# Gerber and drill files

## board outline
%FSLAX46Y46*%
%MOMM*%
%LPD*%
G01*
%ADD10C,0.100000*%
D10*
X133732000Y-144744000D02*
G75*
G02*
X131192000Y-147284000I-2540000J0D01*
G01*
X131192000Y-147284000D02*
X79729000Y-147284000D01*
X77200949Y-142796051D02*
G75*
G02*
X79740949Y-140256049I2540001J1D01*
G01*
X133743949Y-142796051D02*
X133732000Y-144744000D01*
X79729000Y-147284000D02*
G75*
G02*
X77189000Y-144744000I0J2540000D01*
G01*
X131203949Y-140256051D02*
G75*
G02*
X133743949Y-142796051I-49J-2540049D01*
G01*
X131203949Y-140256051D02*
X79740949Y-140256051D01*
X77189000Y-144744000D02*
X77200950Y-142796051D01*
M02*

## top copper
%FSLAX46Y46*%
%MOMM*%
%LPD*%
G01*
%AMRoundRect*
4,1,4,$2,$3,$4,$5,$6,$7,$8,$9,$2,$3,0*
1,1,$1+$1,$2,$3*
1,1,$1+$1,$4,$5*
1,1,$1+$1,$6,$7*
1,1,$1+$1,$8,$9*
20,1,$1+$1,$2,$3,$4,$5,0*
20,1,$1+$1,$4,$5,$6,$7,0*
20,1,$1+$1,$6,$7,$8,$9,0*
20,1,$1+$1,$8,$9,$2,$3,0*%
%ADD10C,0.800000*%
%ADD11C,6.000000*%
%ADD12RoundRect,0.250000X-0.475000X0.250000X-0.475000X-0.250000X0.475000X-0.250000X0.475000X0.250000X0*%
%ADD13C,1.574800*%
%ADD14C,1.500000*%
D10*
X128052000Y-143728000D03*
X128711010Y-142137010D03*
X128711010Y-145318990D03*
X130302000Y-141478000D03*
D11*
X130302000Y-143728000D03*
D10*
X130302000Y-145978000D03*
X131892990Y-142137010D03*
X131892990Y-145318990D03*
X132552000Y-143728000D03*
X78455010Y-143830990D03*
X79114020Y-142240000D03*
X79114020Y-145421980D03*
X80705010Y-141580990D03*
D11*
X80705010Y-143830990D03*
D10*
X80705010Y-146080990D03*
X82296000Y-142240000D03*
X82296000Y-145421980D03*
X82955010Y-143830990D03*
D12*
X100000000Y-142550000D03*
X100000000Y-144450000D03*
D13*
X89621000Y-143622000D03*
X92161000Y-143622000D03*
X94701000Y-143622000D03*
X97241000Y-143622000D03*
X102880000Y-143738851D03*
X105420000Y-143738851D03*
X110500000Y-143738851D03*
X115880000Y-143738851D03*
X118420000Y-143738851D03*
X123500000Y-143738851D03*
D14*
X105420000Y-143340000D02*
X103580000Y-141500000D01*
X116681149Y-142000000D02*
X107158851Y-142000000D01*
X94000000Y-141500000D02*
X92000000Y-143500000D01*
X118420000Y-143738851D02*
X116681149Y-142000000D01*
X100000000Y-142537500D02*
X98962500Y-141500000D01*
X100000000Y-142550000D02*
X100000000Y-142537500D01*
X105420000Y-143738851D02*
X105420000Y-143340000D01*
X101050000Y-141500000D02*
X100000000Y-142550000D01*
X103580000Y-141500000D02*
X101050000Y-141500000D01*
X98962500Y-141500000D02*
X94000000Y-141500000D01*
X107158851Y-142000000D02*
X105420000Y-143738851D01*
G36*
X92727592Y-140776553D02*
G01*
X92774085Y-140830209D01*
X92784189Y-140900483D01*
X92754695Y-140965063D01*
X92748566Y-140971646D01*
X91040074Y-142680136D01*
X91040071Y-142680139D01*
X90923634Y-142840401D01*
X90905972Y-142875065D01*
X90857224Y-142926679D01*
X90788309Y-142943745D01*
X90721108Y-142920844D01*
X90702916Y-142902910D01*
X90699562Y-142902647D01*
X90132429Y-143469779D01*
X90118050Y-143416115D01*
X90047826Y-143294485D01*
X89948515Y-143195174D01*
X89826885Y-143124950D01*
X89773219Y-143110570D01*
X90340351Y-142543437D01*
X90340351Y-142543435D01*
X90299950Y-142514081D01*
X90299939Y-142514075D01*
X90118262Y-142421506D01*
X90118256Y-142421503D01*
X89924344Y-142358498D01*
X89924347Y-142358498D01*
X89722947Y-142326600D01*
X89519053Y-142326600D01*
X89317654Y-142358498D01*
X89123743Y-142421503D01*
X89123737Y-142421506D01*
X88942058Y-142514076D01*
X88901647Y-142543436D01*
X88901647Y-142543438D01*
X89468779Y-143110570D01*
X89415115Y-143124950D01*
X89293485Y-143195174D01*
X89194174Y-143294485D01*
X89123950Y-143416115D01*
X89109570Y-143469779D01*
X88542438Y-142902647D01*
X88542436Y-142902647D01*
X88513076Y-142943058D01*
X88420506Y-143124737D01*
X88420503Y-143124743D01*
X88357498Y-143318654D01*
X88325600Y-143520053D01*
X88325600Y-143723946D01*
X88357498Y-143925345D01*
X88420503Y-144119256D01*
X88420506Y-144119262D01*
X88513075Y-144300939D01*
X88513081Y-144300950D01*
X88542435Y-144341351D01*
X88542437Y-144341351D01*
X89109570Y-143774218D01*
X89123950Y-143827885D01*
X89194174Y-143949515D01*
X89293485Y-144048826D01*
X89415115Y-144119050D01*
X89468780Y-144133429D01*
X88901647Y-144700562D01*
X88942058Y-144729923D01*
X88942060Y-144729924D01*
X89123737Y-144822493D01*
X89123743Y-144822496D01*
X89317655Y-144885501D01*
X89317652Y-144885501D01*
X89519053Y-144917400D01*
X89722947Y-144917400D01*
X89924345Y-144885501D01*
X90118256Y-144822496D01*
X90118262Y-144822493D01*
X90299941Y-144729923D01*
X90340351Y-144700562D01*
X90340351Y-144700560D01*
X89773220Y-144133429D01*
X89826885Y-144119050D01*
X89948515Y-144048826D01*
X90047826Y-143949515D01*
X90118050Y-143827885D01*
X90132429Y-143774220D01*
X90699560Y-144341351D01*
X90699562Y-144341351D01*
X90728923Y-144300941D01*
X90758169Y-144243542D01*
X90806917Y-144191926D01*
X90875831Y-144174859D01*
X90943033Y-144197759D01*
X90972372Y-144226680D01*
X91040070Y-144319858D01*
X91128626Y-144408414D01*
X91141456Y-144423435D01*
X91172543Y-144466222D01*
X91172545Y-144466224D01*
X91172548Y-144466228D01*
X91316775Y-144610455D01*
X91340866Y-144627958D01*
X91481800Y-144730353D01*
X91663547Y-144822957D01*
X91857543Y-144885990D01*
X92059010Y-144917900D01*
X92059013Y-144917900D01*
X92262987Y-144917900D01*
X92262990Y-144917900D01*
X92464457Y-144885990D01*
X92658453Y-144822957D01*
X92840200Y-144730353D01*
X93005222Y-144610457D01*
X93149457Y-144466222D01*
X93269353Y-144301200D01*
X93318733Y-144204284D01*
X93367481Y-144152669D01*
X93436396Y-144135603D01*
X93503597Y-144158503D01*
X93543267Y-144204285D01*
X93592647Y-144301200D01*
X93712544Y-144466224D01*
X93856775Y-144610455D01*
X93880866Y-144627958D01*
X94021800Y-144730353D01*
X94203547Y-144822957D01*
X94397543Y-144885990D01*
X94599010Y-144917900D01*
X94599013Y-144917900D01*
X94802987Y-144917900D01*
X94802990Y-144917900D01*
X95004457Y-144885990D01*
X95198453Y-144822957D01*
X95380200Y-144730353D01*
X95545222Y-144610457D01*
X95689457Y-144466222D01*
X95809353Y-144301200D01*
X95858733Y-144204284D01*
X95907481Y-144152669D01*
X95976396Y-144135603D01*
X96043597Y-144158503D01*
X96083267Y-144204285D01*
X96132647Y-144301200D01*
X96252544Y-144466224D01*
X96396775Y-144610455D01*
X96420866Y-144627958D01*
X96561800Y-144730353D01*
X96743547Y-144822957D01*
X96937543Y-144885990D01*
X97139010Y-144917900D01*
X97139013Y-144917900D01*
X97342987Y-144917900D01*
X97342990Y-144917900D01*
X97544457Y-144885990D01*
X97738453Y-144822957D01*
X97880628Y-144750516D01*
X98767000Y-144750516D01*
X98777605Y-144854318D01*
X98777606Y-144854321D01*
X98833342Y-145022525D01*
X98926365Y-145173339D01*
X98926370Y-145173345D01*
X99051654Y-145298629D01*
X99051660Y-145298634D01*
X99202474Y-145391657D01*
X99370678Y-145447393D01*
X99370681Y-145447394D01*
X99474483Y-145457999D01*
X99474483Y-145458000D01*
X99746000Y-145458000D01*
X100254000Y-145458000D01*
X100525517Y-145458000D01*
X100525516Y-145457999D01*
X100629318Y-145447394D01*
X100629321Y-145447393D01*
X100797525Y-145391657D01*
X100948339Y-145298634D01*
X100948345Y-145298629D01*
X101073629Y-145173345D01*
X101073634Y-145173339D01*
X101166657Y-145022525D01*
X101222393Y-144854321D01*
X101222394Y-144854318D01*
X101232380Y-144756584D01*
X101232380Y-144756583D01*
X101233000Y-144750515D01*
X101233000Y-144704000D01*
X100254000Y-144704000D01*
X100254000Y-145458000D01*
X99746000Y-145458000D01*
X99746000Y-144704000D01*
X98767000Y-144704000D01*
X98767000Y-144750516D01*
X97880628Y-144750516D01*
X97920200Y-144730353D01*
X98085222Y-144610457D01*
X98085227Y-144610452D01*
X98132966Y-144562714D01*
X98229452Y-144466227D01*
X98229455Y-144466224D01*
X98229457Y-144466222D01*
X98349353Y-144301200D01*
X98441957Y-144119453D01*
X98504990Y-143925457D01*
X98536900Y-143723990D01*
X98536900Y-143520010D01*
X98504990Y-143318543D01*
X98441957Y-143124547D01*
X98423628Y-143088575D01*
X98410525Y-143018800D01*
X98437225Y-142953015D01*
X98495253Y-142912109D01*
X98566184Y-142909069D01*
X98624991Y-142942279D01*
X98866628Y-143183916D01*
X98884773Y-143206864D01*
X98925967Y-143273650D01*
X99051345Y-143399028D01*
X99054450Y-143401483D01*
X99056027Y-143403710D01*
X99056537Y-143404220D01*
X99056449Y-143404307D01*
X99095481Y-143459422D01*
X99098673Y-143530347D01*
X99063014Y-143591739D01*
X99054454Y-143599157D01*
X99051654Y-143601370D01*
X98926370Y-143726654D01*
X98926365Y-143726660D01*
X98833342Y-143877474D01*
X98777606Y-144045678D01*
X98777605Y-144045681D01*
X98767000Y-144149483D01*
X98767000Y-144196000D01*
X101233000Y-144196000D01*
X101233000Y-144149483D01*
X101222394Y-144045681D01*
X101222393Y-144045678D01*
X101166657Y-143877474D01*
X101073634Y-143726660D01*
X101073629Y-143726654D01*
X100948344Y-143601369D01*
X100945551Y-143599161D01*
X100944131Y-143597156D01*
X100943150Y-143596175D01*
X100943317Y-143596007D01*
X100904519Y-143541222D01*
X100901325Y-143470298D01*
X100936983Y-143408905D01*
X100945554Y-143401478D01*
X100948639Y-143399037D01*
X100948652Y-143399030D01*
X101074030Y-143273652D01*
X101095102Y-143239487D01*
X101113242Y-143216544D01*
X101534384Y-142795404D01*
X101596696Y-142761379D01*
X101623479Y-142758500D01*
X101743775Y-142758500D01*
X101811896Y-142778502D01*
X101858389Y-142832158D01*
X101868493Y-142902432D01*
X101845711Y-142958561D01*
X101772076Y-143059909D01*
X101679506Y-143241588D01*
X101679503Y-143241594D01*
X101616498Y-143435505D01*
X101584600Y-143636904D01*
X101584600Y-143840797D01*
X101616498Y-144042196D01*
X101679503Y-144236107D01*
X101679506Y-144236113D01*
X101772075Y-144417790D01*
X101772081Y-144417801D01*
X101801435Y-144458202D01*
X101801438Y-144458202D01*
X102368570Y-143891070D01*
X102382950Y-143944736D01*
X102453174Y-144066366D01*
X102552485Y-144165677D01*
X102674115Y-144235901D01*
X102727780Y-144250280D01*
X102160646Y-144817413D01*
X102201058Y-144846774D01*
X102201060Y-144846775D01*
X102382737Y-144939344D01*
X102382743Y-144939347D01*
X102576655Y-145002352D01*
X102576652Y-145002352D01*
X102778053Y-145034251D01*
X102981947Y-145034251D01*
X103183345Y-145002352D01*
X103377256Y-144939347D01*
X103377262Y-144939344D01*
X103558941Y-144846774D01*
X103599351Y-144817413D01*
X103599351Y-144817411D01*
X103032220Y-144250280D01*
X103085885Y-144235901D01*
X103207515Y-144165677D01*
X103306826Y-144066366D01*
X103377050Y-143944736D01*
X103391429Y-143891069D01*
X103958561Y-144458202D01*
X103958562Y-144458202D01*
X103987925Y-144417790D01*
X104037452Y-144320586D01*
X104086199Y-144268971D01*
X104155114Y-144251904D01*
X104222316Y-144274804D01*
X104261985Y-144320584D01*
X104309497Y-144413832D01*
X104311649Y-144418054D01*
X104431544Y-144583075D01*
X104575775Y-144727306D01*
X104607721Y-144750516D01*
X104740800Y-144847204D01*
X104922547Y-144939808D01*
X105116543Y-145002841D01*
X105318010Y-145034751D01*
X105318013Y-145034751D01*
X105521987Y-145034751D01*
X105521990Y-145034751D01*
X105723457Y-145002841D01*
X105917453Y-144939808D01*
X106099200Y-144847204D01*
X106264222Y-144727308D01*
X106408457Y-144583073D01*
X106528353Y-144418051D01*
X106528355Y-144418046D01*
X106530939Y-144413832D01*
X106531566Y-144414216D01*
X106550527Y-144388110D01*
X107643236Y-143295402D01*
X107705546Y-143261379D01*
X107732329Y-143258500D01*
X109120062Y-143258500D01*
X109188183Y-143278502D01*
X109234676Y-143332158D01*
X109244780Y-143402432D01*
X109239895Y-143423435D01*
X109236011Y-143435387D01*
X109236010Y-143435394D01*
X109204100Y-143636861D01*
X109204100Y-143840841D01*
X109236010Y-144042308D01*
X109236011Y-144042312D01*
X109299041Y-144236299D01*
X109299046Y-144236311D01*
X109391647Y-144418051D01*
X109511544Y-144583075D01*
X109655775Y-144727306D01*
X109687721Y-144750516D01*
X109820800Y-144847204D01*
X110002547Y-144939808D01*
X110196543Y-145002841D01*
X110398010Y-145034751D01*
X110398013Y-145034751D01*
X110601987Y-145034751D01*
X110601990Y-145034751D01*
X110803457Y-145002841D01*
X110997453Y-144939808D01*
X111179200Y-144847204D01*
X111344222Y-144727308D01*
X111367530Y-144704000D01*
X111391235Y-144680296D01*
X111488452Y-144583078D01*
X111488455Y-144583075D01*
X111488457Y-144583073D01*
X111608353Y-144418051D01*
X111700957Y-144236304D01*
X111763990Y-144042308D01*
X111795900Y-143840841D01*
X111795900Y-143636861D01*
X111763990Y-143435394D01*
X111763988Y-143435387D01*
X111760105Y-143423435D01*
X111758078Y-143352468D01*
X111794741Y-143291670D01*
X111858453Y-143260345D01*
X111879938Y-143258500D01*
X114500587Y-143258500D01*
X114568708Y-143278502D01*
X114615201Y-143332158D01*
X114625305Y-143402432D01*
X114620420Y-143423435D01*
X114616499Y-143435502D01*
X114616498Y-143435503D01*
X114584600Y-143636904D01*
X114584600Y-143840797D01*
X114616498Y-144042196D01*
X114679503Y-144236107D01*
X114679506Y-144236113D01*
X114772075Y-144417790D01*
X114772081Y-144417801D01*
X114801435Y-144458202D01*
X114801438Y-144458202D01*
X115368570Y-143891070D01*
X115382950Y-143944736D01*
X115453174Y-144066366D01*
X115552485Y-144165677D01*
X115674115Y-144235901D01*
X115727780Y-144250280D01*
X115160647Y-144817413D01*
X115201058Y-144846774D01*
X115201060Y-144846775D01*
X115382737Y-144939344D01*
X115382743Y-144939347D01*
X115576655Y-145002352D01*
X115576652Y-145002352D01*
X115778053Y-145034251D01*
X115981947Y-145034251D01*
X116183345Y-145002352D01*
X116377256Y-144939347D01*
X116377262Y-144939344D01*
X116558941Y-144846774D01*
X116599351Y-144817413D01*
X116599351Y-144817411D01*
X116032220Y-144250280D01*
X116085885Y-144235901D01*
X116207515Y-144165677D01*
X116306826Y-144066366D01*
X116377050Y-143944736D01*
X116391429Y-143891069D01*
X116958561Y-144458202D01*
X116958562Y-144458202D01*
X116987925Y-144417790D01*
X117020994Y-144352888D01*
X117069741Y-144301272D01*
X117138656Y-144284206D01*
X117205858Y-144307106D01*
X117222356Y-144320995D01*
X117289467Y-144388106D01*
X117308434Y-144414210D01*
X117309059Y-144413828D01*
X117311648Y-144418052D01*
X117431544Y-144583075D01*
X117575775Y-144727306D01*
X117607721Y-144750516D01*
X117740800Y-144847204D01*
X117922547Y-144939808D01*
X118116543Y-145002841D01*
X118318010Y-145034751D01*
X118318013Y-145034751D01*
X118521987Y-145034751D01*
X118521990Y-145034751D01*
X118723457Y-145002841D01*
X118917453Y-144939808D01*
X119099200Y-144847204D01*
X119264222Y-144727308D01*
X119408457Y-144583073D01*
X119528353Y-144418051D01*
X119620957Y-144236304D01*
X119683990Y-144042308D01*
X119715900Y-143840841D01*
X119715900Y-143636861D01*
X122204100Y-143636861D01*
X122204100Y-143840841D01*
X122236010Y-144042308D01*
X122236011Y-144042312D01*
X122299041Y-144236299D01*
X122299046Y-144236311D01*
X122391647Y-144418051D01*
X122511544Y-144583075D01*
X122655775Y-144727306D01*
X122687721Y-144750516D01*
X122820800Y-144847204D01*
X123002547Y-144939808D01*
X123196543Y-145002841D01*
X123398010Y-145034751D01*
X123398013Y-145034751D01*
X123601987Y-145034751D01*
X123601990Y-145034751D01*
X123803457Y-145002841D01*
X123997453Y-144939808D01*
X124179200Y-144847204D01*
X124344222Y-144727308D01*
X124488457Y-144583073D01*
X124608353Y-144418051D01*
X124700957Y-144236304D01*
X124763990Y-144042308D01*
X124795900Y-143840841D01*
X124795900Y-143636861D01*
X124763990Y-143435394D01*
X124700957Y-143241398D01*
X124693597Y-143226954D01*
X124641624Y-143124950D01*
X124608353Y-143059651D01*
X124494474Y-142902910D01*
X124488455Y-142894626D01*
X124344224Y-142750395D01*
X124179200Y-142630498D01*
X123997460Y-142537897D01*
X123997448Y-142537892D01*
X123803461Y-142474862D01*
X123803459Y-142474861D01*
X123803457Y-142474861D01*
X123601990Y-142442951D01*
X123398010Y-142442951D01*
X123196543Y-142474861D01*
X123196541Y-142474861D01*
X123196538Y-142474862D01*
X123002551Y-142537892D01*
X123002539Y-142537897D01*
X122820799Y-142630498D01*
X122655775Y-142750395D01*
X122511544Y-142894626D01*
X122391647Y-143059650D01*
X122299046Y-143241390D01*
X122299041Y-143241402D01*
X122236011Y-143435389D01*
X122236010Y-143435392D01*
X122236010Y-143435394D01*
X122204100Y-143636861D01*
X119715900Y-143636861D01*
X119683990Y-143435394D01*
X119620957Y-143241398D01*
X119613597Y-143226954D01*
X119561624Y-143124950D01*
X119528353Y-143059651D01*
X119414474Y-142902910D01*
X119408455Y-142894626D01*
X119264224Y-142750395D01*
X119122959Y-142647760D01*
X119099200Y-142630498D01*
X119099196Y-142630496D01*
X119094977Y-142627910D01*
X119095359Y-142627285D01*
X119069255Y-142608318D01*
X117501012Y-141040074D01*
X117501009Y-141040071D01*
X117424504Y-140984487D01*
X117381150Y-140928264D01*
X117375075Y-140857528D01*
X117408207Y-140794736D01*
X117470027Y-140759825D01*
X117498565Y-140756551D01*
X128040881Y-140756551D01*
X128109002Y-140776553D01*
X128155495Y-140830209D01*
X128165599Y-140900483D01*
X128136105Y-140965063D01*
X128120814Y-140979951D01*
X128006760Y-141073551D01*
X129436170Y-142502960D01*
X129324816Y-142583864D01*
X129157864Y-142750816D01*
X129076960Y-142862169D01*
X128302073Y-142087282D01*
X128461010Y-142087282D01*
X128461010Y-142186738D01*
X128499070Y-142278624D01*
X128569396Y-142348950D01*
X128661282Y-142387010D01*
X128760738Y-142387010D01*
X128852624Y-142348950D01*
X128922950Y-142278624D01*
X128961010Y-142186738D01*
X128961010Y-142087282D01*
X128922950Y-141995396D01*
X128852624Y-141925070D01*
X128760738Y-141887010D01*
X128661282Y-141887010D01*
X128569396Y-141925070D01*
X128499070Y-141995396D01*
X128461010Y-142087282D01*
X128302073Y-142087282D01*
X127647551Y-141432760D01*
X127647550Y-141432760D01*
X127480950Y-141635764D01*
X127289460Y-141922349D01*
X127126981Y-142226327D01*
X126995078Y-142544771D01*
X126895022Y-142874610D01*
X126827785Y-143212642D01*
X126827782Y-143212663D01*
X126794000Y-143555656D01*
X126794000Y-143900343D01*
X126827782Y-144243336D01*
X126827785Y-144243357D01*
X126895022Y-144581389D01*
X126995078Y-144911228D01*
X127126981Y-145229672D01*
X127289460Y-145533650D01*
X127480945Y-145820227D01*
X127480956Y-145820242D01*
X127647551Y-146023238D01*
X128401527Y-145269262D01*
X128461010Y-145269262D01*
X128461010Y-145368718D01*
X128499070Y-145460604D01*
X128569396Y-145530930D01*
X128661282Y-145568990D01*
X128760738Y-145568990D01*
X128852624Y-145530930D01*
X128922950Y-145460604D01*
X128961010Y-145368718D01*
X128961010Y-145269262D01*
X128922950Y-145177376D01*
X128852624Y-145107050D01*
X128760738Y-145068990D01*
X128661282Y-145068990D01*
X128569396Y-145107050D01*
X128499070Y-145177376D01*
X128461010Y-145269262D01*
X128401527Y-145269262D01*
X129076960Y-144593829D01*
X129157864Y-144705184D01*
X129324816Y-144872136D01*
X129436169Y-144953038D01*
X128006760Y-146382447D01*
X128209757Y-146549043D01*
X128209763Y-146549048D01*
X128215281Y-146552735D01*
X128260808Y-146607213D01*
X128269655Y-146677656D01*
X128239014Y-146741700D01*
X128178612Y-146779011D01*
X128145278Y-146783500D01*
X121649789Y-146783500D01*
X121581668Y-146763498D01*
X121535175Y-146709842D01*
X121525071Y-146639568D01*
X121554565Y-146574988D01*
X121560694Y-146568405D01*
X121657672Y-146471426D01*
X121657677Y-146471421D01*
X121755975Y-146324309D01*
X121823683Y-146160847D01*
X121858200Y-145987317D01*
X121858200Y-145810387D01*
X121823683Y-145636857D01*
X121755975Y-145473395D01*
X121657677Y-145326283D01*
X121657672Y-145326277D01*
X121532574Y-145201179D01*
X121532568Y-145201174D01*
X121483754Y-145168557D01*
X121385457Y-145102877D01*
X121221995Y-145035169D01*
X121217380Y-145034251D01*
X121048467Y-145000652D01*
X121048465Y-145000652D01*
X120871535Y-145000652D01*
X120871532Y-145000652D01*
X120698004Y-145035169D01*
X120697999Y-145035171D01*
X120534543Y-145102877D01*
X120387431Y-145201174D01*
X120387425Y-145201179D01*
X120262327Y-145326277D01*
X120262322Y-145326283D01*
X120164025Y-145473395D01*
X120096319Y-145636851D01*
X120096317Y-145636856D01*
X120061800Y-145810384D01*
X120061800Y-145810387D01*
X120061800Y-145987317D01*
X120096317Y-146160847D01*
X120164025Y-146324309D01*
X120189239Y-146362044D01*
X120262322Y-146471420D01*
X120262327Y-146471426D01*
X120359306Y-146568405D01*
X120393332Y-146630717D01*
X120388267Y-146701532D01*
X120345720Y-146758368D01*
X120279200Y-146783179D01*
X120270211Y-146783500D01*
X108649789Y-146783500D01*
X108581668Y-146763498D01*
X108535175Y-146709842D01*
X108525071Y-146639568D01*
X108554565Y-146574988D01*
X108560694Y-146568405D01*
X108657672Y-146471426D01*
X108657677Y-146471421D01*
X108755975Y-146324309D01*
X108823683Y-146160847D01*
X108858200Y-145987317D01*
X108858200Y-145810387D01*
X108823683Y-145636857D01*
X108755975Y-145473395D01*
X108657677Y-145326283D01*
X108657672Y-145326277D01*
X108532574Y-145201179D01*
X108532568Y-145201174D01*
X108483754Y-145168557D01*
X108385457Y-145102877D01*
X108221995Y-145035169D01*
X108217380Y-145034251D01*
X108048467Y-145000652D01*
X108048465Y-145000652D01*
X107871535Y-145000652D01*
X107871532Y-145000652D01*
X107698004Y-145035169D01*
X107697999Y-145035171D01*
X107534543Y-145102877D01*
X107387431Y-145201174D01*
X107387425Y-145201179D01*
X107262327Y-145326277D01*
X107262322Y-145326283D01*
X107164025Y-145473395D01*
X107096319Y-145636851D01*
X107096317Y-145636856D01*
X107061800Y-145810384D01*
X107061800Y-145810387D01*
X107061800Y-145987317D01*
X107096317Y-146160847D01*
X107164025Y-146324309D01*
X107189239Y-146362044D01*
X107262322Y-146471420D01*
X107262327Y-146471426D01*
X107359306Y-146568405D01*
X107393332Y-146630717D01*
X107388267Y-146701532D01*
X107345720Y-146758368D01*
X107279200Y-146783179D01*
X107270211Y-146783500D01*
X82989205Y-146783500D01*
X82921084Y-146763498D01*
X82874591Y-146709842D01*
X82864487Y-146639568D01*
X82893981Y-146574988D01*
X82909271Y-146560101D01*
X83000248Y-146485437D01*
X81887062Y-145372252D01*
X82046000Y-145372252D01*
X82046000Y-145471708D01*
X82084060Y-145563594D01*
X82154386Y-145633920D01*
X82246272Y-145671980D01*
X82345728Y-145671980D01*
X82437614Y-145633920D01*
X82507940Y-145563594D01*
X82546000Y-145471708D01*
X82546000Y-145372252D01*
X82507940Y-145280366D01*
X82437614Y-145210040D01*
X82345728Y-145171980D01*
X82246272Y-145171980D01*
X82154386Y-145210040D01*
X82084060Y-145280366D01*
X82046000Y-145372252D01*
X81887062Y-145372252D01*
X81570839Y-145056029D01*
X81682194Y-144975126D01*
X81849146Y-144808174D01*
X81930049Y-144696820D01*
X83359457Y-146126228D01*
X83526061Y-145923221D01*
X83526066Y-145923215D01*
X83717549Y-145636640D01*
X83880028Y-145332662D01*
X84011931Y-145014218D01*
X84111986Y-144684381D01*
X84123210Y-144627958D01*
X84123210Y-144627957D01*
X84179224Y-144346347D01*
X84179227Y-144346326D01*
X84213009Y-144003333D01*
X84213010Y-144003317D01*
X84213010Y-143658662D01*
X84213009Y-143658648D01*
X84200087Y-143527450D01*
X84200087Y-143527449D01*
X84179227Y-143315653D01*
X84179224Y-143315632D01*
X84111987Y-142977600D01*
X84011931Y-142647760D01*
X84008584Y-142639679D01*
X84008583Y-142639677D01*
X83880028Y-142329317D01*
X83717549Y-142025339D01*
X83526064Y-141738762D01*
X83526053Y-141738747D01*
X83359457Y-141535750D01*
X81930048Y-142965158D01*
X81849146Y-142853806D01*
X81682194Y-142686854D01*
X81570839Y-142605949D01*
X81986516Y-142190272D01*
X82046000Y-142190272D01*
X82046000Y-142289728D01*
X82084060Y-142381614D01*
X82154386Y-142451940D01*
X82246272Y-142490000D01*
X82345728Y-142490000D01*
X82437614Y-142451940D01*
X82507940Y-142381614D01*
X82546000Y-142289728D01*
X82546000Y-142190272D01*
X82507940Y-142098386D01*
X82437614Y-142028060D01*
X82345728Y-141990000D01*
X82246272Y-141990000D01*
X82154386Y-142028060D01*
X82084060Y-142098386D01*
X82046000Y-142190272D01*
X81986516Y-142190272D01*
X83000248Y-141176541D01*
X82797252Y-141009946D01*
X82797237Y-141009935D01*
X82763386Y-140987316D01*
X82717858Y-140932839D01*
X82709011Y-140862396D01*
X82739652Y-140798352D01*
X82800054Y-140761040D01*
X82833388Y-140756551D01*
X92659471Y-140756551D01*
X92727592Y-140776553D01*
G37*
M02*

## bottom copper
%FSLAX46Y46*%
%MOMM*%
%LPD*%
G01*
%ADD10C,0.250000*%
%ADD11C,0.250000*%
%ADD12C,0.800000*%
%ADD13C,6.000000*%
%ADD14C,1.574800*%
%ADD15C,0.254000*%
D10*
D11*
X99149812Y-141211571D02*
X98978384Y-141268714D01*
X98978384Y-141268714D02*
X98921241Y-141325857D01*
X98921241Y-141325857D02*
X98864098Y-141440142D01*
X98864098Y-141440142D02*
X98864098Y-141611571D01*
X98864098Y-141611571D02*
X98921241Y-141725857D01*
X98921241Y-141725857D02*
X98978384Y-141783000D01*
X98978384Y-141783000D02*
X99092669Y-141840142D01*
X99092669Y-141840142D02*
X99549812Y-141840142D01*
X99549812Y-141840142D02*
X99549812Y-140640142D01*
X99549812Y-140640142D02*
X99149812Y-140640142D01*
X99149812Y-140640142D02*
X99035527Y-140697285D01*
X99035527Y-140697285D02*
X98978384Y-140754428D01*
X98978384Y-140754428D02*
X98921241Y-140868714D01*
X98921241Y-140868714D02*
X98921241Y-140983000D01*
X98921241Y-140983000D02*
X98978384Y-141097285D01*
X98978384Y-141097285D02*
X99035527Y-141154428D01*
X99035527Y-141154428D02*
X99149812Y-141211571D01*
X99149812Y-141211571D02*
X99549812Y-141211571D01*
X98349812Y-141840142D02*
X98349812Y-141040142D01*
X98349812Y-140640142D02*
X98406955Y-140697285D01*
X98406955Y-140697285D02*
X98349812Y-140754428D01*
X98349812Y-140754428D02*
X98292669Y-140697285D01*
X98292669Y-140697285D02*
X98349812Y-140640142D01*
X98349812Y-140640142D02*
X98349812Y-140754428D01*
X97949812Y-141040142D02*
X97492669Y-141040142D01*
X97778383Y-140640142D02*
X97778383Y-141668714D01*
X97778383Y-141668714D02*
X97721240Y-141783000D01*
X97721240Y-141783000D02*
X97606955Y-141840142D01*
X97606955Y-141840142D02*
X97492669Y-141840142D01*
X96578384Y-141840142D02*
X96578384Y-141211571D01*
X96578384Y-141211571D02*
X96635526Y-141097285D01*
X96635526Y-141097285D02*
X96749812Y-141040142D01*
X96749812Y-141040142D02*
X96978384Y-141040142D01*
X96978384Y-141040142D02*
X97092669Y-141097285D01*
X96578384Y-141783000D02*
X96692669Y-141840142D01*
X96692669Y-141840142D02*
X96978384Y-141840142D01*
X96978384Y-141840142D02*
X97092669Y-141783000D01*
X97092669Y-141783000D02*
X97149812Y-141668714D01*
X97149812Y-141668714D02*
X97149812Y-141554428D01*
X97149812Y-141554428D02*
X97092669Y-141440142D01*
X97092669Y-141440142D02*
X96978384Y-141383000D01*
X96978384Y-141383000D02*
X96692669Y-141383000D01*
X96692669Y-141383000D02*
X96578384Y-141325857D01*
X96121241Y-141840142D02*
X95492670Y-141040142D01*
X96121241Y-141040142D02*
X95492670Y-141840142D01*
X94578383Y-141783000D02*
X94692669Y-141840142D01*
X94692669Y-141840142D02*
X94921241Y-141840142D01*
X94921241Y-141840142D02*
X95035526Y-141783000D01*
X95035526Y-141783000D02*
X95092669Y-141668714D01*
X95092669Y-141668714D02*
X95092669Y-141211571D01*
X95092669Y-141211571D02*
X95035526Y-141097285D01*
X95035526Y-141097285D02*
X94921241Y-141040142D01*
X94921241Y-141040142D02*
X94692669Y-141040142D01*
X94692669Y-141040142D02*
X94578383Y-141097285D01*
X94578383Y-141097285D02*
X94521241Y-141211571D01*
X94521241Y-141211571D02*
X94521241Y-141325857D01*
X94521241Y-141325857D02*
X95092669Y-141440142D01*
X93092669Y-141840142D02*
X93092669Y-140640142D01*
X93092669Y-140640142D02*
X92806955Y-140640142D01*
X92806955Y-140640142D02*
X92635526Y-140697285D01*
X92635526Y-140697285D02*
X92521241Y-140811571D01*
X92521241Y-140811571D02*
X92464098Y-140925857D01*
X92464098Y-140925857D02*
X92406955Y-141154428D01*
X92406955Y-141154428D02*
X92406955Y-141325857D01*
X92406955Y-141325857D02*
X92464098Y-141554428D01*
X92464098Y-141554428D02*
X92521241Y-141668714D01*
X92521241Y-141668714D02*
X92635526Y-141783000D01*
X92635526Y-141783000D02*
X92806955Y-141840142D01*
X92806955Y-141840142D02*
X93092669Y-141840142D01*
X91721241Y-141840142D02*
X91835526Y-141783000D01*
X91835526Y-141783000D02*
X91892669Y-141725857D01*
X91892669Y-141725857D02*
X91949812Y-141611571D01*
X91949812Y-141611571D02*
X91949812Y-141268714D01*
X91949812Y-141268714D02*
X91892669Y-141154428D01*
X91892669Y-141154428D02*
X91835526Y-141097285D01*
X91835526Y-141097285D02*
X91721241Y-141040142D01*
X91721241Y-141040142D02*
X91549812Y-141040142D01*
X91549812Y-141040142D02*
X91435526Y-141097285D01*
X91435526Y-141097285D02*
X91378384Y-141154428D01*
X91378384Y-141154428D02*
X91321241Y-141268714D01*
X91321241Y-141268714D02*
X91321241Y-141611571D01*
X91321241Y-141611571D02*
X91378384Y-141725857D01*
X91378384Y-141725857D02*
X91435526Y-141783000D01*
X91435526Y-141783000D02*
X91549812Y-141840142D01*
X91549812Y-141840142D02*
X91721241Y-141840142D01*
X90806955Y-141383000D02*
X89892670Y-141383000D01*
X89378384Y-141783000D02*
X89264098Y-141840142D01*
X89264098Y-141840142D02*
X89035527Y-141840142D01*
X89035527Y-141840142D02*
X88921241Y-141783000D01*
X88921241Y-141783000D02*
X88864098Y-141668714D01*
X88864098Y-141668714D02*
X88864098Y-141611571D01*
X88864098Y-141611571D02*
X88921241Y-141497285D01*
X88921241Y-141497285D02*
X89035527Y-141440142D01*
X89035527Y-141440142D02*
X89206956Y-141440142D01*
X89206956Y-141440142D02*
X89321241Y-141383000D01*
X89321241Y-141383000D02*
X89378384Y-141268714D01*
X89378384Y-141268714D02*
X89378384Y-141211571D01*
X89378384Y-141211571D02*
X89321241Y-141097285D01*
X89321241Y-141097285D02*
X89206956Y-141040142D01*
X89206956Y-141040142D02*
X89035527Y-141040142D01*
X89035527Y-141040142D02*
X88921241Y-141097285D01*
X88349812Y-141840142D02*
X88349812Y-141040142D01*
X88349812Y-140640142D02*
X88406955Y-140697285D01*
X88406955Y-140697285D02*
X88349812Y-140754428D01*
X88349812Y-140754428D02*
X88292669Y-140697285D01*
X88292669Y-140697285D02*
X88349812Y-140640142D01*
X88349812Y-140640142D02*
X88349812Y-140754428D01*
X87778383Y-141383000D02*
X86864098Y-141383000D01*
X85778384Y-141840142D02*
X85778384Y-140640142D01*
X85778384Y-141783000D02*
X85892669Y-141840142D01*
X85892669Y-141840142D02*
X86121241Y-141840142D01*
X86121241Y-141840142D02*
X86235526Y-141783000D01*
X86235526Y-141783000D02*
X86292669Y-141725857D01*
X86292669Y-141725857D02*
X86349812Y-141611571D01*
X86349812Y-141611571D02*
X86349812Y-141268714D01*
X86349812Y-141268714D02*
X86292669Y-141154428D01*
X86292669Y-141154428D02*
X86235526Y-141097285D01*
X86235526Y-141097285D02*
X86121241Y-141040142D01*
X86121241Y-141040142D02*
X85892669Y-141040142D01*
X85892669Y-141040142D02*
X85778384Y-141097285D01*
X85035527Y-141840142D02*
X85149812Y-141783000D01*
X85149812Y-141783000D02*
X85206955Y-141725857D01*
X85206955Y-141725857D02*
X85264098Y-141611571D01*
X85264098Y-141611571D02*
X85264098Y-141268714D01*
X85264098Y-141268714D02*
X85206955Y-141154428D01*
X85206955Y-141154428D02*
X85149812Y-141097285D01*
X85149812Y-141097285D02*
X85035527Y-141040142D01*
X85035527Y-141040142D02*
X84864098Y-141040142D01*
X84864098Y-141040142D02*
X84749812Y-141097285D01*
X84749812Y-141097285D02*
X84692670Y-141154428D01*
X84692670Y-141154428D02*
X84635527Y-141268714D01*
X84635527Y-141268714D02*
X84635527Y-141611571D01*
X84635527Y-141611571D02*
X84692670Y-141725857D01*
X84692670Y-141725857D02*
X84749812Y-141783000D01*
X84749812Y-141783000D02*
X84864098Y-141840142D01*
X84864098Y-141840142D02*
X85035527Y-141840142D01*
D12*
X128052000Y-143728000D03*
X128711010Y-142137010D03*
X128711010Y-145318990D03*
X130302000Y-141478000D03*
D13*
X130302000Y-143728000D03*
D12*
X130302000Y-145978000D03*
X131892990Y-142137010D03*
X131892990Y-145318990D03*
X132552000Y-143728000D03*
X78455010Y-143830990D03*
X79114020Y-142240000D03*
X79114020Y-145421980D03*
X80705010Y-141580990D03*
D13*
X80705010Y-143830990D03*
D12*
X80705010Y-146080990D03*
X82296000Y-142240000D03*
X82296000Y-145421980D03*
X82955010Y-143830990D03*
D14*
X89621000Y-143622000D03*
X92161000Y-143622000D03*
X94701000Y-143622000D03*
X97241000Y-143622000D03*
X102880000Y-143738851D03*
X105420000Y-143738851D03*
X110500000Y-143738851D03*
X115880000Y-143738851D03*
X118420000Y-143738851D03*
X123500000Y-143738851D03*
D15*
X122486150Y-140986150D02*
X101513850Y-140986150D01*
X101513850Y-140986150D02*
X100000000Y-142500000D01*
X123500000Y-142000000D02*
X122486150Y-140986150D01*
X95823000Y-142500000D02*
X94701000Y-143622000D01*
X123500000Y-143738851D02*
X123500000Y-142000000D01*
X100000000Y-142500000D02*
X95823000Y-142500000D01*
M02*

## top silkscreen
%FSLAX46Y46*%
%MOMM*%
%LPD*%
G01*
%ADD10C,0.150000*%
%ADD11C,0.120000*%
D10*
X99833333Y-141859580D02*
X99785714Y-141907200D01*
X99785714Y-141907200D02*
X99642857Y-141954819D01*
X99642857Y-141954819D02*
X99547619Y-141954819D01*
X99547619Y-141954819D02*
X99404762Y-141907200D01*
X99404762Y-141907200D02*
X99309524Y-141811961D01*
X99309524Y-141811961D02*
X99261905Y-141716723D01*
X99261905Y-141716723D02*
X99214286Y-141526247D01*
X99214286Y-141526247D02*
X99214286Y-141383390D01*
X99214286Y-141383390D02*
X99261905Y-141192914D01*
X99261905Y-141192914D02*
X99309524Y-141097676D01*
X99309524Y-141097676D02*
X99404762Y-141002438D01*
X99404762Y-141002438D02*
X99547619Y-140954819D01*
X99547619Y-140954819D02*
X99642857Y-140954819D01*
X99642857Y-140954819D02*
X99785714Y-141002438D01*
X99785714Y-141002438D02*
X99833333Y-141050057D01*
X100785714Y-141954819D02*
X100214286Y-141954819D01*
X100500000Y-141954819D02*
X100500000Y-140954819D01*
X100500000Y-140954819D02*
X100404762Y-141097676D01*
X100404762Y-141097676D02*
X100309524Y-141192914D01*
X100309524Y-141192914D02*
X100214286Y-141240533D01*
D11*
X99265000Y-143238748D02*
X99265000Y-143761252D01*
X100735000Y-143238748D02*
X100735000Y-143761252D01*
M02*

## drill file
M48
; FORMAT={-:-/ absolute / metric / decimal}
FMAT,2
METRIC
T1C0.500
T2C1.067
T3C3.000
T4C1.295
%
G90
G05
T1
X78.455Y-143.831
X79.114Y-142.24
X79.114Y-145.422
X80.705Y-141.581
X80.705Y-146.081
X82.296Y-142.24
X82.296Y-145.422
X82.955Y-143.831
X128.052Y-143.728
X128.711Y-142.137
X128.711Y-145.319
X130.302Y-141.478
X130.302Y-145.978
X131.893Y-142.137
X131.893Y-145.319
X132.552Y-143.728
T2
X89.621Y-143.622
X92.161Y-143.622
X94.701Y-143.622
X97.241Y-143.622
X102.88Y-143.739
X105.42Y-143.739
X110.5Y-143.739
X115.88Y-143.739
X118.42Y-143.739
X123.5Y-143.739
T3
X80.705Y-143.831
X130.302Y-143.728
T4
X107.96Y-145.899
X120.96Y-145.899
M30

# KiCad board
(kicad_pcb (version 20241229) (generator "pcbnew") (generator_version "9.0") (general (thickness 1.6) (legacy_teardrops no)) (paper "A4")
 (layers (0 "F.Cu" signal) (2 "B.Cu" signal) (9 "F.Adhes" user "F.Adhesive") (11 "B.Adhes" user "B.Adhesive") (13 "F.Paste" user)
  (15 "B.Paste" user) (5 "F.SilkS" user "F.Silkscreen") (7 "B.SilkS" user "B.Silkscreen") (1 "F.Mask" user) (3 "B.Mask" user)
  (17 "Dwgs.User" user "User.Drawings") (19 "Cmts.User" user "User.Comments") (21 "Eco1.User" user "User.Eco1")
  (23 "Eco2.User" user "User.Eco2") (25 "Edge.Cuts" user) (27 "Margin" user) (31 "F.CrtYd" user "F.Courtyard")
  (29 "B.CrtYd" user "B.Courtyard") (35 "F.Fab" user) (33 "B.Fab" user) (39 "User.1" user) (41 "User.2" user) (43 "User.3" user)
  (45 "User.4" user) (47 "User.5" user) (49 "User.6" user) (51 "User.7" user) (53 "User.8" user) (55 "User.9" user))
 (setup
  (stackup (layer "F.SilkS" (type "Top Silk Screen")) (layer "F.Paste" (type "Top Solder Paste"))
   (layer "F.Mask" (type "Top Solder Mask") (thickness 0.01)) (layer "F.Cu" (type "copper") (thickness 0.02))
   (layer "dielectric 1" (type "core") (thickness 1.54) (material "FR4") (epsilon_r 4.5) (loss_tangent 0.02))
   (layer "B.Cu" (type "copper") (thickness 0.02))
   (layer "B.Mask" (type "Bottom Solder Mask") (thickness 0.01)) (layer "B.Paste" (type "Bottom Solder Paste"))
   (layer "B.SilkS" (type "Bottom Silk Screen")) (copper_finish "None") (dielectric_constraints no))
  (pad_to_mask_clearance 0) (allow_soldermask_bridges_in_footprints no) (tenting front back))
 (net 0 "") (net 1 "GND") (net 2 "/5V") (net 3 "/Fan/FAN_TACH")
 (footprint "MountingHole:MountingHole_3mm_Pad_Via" (layer "F.Cu") (at 130.302 143.728)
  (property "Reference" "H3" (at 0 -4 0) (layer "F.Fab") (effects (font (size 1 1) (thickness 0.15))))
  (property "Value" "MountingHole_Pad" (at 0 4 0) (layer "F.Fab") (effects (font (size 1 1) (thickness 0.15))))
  (pad "1" thru_hole circle (at -2.25 0) (size 0.8 0.8) (drill 0.5) (layers "*.Cu" "*.Mask") (remove_unused_layers no) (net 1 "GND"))
  (pad "1" thru_hole circle (at -1.59099 -1.59099) (size 0.8 0.8) (drill 0.5) (layers "*.Cu" "*.Mask") (remove_unused_layers no)
   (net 1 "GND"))
  (pad "1" thru_hole circle (at -1.59099 1.59099) (size 0.8 0.8) (drill 0.5) (layers "*.Cu" "*.Mask") (remove_unused_layers no)
   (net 1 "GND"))
  (pad "1" thru_hole circle (at 0 -2.25) (size 0.8 0.8) (drill 0.5) (layers "*.Cu" "*.Mask") (remove_unused_layers no) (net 1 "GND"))
  (pad "1" thru_hole circle (at 0 0) (size 6 6) (drill 3) (layers "*.Cu" "*.Mask") (remove_unused_layers no) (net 1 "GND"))
  (pad "1" thru_hole circle (at 0 2.25) (size 0.8 0.8) (drill 0.5) (layers "*.Cu" "*.Mask") (remove_unused_layers no) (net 1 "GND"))
  (pad "1" thru_hole circle (at 1.59099 -1.59099) (size 0.8 0.8) (drill 0.5) (layers "*.Cu" "*.Mask") (remove_unused_layers no)
   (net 1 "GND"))
  (pad "1" thru_hole circle (at 1.59099 1.59099) (size 0.8 0.8) (drill 0.5) (layers "*.Cu" "*.Mask") (remove_unused_layers no) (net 1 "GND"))
  (pad "1" thru_hole circle (at 2.25 0) (size 0.8 0.8) (drill 0.5) (layers "*.Cu" "*.Mask") (remove_unused_layers no) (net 1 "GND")))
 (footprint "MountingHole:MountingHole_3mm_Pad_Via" (layer "F.Cu") (at 80.70501 143.83099)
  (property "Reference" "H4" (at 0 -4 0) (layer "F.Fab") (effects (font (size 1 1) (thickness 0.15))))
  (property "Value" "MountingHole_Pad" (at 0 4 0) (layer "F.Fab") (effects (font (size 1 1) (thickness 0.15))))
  (pad "1" thru_hole circle (at -2.25 0) (size 0.8 0.8) (drill 0.5) (layers "*.Cu" "*.Mask") (remove_unused_layers no) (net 1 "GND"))
  (pad "1" thru_hole circle (at -1.59099 -1.59099) (size 0.8 0.8) (drill 0.5) (layers "*.Cu" "*.Mask") (remove_unused_layers no)
   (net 1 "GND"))
  (pad "1" thru_hole circle (at -1.59099 1.59099) (size 0.8 0.8) (drill 0.5) (layers "*.Cu" "*.Mask") (remove_unused_layers no)
   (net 1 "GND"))
  (pad "1" thru_hole circle (at 0 -2.25) (size 0.8 0.8) (drill 0.5) (layers "*.Cu" "*.Mask") (remove_unused_layers no) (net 1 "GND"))
  (pad "1" thru_hole circle (at 0 0) (size 6 6) (drill 3) (layers "*.Cu" "*.Mask") (remove_unused_layers no) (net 1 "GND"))
  (pad "1" thru_hole circle (at 0 2.25) (size 0.8 0.8) (drill 0.5) (layers "*.Cu" "*.Mask") (remove_unused_layers no) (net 1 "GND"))
  (pad "1" thru_hole circle (at 1.59099 -1.59099) (size 0.8 0.8) (drill 0.5) (layers "*.Cu" "*.Mask") (remove_unused_layers no)
   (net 1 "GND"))
  (pad "1" thru_hole circle (at 1.59099 1.59099) (size 0.8 0.8) (drill 0.5) (layers "*.Cu" "*.Mask") (remove_unused_layers no) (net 1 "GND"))
  (pad "1" thru_hole circle (at 2.25 0) (size 0.8 0.8) (drill 0.5) (layers "*.Cu" "*.Mask") (remove_unused_layers no) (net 1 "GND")))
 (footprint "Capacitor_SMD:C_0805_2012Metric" (layer "F.Cu") (at 100 143.5 -90)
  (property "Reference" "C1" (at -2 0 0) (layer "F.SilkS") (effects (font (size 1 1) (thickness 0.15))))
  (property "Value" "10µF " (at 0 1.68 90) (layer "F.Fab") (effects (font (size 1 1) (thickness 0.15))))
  (fp_line (start -0.261252 0.735) (end 0.261252 0.735) (stroke (width 0.12) (type solid)) (layer "F.SilkS"))
  (fp_line (start -0.261252 -0.735) (end 0.261252 -0.735) (stroke (width 0.12) (type solid)) (layer "F.SilkS"))
  (pad "1" smd roundrect (at -0.95 0 270) (size 1 1.45) (layers "F.Cu" "F.Mask" "F.Paste") (roundrect_rratio 0.25) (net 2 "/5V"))
  (pad "2" smd roundrect (at 0.95 0 270) (size 1 1.45) (layers "F.Cu" "F.Mask" "F.Paste") (roundrect_rratio 0.25) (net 1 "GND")))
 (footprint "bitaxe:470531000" (layer "B.Cu") (at 89.621 143.622)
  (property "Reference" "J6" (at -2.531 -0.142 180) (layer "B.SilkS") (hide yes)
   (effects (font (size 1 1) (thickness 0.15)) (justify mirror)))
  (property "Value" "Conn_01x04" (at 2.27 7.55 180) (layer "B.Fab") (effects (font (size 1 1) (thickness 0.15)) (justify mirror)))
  (pad "1" thru_hole circle (at 0 0) (size 1.5748 1.5748) (drill 1.0668) (layers "*.Cu" "*.Mask") (remove_unused_layers no) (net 1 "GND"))
  (pad "2" thru_hole circle (at 2.54 0) (size 1.5748 1.5748) (drill 1.0668) (layers "*.Cu" "*.Mask") (remove_unused_layers no) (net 2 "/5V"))
  (pad "3" thru_hole circle (at 5.08 0) (size 1.5748 1.5748) (drill 1.0668) (layers "*.Cu" "*.Mask") (remove_unused_layers no)
   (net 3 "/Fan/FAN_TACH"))
  (pad "4" thru_hole circle (at 7.62 0) (size 1.5748 1.5748) (drill 1.0668) (layers "*.Cu" "*.Mask") (remove_unused_layers no)))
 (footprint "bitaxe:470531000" (layer "B.Cu") (at 102.88 143.738851)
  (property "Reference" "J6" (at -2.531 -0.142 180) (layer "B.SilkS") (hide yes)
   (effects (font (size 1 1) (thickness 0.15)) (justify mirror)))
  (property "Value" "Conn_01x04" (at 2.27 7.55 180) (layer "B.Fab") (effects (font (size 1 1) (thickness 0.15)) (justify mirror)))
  (pad "" np_thru_hole circle (at 5.08 2.160001 270) (size 1.2954 1.2954) (drill 1.2954) (layers "*.Cu" "*.Mask"))
  (pad "1" thru_hole circle (at 0 0) (size 1.5748 1.5748) (drill 1.0668) (layers "*.Cu" "*.Mask") (remove_unused_layers no) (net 1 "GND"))
  (pad "2" thru_hole circle (at 2.54 0) (size 1.5748 1.5748) (drill 1.0668) (layers "*.Cu" "*.Mask") (remove_unused_layers no) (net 2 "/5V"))
  (pad "4" thru_hole circle (at 7.62 0) (size 1.5748 1.5748) (drill 1.0668) (layers "*.Cu" "*.Mask") (remove_unused_layers no)))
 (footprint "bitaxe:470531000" (layer "B.Cu") (at 115.88 143.738851)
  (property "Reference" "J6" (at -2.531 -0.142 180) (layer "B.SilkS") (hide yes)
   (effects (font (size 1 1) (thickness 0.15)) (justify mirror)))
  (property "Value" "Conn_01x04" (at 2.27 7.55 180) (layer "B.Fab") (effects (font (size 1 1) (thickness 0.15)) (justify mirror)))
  (pad "" np_thru_hole circle (at 5.08 2.160001 270) (size 1.2954 1.2954) (drill 1.2954) (layers "*.Cu" "*.Mask"))
  (pad "1" thru_hole circle (at 0 0) (size 1.5748 1.5748) (drill 1.0668) (layers "*.Cu" "*.Mask") (remove_unused_layers no) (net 1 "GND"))
  (pad "2" thru_hole circle (at 2.54 0) (size 1.5748 1.5748) (drill 1.0668) (layers "*.Cu" "*.Mask") (remove_unused_layers no) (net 2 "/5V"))
  (pad "4" thru_hole circle (at 7.62 0) (size 1.5748 1.5748) (drill 1.0668) (layers "*.Cu" "*.Mask") (remove_unused_layers no)
   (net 3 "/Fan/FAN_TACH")))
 (gr_arc (start 133.732 144.744) (mid 132.988051 146.540051) (end 131.192 147.284) (stroke (width 0.1) (type default)) (layer "Edge.Cuts"))
 (gr_line (start 131.192 147.284) (end 79.729 147.284) (stroke (width 0.1) (type default)) (layer "Edge.Cuts"))
 (gr_arc (start 77.200949 142.796051) (mid 77.944898 141) (end 79.740949 140.256051) (stroke (width 0.1) (type default)) (layer "Edge.Cuts"))
 (gr_line (start 133.743949 142.796051) (end 133.732 144.744) (stroke (width 0.1) (type default)) (layer "Edge.Cuts"))
 (gr_arc (start 79.729 147.284) (mid 77.932949 146.540051) (end 77.189 144.744) (stroke (width 0.1) (type default)) (layer "Edge.Cuts"))
 (gr_arc (start 131.203949 140.256051) (mid 133 141) (end 133.743949 142.796051) (stroke (width 0.1) (type default)) (layer "Edge.Cuts"))
 (gr_line (start 131.203949 140.256051) (end 79.740949 140.256051) (stroke (width 0.1) (type default)) (layer "Edge.Cuts"))
 (gr_line (start 77.189 144.744) (end 77.20095 142.796051) (stroke (width 0.1) (type default)) (layer "Edge.Cuts"))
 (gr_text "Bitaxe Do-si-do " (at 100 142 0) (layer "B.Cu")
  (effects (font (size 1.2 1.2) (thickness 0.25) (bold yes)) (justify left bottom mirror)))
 (segment (start 105.42 143.34) (end 103.58 141.5) (width 1.5) (layer "F.Cu") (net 2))
 (segment (start 116.681149 142) (end 107.158851 142) (width 1.5) (layer "F.Cu") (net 2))
 (segment (start 94 141.5) (end 92 143.5) (width 1.5) (layer "F.Cu") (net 2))
 (segment (start 118.42 143.738851) (end 116.681149 142) (width 1.5) (layer "F.Cu") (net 2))
 (segment (start 100 142.5375) (end 98.9625 141.5) (width 1.5) (layer "F.Cu") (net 2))
 (segment (start 100 142.55) (end 100 142.5375) (width 1.5) (layer "F.Cu") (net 2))
 (segment (start 105.42 143.738851) (end 105.42 143.34) (width 1.5) (layer "F.Cu") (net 2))
 (segment (start 101.05 141.5) (end 100 142.55) (width 1.5) (layer "F.Cu") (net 2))
 (segment (start 103.58 141.5) (end 101.05 141.5) (width 1.5) (layer "F.Cu") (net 2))
 (segment (start 98.9625 141.5) (end 94 141.5) (width 1.5) (layer "F.Cu") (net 2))
 (segment (start 107.158851 142) (end 105.42 143.738851) (width 1.5) (layer "F.Cu") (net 2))
 (segment (start 122.48615 140.98615) (end 101.51385 140.98615) (width 0.254) (layer "B.Cu") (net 3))
 (segment (start 101.51385 140.98615) (end 100 142.5) (width 0.254) (layer "B.Cu") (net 3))
 (segment (start 123.5 142) (end 122.48615 140.98615) (width 0.254) (layer "B.Cu") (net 3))
 (segment (start 95.823 142.5) (end 94.701 143.622) (width 0.254) (layer "B.Cu") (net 3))
 (segment (start 123.5 143.738851) (end 123.5 142) (width 0.254) (layer "B.Cu") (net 3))
 (segment (start 100 142.5) (end 95.823 142.5) (width 0.254) (layer "B.Cu") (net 3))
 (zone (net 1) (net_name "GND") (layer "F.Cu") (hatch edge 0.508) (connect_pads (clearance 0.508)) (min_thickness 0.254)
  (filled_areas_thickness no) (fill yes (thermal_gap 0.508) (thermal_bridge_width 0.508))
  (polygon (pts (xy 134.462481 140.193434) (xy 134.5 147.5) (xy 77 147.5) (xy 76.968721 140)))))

